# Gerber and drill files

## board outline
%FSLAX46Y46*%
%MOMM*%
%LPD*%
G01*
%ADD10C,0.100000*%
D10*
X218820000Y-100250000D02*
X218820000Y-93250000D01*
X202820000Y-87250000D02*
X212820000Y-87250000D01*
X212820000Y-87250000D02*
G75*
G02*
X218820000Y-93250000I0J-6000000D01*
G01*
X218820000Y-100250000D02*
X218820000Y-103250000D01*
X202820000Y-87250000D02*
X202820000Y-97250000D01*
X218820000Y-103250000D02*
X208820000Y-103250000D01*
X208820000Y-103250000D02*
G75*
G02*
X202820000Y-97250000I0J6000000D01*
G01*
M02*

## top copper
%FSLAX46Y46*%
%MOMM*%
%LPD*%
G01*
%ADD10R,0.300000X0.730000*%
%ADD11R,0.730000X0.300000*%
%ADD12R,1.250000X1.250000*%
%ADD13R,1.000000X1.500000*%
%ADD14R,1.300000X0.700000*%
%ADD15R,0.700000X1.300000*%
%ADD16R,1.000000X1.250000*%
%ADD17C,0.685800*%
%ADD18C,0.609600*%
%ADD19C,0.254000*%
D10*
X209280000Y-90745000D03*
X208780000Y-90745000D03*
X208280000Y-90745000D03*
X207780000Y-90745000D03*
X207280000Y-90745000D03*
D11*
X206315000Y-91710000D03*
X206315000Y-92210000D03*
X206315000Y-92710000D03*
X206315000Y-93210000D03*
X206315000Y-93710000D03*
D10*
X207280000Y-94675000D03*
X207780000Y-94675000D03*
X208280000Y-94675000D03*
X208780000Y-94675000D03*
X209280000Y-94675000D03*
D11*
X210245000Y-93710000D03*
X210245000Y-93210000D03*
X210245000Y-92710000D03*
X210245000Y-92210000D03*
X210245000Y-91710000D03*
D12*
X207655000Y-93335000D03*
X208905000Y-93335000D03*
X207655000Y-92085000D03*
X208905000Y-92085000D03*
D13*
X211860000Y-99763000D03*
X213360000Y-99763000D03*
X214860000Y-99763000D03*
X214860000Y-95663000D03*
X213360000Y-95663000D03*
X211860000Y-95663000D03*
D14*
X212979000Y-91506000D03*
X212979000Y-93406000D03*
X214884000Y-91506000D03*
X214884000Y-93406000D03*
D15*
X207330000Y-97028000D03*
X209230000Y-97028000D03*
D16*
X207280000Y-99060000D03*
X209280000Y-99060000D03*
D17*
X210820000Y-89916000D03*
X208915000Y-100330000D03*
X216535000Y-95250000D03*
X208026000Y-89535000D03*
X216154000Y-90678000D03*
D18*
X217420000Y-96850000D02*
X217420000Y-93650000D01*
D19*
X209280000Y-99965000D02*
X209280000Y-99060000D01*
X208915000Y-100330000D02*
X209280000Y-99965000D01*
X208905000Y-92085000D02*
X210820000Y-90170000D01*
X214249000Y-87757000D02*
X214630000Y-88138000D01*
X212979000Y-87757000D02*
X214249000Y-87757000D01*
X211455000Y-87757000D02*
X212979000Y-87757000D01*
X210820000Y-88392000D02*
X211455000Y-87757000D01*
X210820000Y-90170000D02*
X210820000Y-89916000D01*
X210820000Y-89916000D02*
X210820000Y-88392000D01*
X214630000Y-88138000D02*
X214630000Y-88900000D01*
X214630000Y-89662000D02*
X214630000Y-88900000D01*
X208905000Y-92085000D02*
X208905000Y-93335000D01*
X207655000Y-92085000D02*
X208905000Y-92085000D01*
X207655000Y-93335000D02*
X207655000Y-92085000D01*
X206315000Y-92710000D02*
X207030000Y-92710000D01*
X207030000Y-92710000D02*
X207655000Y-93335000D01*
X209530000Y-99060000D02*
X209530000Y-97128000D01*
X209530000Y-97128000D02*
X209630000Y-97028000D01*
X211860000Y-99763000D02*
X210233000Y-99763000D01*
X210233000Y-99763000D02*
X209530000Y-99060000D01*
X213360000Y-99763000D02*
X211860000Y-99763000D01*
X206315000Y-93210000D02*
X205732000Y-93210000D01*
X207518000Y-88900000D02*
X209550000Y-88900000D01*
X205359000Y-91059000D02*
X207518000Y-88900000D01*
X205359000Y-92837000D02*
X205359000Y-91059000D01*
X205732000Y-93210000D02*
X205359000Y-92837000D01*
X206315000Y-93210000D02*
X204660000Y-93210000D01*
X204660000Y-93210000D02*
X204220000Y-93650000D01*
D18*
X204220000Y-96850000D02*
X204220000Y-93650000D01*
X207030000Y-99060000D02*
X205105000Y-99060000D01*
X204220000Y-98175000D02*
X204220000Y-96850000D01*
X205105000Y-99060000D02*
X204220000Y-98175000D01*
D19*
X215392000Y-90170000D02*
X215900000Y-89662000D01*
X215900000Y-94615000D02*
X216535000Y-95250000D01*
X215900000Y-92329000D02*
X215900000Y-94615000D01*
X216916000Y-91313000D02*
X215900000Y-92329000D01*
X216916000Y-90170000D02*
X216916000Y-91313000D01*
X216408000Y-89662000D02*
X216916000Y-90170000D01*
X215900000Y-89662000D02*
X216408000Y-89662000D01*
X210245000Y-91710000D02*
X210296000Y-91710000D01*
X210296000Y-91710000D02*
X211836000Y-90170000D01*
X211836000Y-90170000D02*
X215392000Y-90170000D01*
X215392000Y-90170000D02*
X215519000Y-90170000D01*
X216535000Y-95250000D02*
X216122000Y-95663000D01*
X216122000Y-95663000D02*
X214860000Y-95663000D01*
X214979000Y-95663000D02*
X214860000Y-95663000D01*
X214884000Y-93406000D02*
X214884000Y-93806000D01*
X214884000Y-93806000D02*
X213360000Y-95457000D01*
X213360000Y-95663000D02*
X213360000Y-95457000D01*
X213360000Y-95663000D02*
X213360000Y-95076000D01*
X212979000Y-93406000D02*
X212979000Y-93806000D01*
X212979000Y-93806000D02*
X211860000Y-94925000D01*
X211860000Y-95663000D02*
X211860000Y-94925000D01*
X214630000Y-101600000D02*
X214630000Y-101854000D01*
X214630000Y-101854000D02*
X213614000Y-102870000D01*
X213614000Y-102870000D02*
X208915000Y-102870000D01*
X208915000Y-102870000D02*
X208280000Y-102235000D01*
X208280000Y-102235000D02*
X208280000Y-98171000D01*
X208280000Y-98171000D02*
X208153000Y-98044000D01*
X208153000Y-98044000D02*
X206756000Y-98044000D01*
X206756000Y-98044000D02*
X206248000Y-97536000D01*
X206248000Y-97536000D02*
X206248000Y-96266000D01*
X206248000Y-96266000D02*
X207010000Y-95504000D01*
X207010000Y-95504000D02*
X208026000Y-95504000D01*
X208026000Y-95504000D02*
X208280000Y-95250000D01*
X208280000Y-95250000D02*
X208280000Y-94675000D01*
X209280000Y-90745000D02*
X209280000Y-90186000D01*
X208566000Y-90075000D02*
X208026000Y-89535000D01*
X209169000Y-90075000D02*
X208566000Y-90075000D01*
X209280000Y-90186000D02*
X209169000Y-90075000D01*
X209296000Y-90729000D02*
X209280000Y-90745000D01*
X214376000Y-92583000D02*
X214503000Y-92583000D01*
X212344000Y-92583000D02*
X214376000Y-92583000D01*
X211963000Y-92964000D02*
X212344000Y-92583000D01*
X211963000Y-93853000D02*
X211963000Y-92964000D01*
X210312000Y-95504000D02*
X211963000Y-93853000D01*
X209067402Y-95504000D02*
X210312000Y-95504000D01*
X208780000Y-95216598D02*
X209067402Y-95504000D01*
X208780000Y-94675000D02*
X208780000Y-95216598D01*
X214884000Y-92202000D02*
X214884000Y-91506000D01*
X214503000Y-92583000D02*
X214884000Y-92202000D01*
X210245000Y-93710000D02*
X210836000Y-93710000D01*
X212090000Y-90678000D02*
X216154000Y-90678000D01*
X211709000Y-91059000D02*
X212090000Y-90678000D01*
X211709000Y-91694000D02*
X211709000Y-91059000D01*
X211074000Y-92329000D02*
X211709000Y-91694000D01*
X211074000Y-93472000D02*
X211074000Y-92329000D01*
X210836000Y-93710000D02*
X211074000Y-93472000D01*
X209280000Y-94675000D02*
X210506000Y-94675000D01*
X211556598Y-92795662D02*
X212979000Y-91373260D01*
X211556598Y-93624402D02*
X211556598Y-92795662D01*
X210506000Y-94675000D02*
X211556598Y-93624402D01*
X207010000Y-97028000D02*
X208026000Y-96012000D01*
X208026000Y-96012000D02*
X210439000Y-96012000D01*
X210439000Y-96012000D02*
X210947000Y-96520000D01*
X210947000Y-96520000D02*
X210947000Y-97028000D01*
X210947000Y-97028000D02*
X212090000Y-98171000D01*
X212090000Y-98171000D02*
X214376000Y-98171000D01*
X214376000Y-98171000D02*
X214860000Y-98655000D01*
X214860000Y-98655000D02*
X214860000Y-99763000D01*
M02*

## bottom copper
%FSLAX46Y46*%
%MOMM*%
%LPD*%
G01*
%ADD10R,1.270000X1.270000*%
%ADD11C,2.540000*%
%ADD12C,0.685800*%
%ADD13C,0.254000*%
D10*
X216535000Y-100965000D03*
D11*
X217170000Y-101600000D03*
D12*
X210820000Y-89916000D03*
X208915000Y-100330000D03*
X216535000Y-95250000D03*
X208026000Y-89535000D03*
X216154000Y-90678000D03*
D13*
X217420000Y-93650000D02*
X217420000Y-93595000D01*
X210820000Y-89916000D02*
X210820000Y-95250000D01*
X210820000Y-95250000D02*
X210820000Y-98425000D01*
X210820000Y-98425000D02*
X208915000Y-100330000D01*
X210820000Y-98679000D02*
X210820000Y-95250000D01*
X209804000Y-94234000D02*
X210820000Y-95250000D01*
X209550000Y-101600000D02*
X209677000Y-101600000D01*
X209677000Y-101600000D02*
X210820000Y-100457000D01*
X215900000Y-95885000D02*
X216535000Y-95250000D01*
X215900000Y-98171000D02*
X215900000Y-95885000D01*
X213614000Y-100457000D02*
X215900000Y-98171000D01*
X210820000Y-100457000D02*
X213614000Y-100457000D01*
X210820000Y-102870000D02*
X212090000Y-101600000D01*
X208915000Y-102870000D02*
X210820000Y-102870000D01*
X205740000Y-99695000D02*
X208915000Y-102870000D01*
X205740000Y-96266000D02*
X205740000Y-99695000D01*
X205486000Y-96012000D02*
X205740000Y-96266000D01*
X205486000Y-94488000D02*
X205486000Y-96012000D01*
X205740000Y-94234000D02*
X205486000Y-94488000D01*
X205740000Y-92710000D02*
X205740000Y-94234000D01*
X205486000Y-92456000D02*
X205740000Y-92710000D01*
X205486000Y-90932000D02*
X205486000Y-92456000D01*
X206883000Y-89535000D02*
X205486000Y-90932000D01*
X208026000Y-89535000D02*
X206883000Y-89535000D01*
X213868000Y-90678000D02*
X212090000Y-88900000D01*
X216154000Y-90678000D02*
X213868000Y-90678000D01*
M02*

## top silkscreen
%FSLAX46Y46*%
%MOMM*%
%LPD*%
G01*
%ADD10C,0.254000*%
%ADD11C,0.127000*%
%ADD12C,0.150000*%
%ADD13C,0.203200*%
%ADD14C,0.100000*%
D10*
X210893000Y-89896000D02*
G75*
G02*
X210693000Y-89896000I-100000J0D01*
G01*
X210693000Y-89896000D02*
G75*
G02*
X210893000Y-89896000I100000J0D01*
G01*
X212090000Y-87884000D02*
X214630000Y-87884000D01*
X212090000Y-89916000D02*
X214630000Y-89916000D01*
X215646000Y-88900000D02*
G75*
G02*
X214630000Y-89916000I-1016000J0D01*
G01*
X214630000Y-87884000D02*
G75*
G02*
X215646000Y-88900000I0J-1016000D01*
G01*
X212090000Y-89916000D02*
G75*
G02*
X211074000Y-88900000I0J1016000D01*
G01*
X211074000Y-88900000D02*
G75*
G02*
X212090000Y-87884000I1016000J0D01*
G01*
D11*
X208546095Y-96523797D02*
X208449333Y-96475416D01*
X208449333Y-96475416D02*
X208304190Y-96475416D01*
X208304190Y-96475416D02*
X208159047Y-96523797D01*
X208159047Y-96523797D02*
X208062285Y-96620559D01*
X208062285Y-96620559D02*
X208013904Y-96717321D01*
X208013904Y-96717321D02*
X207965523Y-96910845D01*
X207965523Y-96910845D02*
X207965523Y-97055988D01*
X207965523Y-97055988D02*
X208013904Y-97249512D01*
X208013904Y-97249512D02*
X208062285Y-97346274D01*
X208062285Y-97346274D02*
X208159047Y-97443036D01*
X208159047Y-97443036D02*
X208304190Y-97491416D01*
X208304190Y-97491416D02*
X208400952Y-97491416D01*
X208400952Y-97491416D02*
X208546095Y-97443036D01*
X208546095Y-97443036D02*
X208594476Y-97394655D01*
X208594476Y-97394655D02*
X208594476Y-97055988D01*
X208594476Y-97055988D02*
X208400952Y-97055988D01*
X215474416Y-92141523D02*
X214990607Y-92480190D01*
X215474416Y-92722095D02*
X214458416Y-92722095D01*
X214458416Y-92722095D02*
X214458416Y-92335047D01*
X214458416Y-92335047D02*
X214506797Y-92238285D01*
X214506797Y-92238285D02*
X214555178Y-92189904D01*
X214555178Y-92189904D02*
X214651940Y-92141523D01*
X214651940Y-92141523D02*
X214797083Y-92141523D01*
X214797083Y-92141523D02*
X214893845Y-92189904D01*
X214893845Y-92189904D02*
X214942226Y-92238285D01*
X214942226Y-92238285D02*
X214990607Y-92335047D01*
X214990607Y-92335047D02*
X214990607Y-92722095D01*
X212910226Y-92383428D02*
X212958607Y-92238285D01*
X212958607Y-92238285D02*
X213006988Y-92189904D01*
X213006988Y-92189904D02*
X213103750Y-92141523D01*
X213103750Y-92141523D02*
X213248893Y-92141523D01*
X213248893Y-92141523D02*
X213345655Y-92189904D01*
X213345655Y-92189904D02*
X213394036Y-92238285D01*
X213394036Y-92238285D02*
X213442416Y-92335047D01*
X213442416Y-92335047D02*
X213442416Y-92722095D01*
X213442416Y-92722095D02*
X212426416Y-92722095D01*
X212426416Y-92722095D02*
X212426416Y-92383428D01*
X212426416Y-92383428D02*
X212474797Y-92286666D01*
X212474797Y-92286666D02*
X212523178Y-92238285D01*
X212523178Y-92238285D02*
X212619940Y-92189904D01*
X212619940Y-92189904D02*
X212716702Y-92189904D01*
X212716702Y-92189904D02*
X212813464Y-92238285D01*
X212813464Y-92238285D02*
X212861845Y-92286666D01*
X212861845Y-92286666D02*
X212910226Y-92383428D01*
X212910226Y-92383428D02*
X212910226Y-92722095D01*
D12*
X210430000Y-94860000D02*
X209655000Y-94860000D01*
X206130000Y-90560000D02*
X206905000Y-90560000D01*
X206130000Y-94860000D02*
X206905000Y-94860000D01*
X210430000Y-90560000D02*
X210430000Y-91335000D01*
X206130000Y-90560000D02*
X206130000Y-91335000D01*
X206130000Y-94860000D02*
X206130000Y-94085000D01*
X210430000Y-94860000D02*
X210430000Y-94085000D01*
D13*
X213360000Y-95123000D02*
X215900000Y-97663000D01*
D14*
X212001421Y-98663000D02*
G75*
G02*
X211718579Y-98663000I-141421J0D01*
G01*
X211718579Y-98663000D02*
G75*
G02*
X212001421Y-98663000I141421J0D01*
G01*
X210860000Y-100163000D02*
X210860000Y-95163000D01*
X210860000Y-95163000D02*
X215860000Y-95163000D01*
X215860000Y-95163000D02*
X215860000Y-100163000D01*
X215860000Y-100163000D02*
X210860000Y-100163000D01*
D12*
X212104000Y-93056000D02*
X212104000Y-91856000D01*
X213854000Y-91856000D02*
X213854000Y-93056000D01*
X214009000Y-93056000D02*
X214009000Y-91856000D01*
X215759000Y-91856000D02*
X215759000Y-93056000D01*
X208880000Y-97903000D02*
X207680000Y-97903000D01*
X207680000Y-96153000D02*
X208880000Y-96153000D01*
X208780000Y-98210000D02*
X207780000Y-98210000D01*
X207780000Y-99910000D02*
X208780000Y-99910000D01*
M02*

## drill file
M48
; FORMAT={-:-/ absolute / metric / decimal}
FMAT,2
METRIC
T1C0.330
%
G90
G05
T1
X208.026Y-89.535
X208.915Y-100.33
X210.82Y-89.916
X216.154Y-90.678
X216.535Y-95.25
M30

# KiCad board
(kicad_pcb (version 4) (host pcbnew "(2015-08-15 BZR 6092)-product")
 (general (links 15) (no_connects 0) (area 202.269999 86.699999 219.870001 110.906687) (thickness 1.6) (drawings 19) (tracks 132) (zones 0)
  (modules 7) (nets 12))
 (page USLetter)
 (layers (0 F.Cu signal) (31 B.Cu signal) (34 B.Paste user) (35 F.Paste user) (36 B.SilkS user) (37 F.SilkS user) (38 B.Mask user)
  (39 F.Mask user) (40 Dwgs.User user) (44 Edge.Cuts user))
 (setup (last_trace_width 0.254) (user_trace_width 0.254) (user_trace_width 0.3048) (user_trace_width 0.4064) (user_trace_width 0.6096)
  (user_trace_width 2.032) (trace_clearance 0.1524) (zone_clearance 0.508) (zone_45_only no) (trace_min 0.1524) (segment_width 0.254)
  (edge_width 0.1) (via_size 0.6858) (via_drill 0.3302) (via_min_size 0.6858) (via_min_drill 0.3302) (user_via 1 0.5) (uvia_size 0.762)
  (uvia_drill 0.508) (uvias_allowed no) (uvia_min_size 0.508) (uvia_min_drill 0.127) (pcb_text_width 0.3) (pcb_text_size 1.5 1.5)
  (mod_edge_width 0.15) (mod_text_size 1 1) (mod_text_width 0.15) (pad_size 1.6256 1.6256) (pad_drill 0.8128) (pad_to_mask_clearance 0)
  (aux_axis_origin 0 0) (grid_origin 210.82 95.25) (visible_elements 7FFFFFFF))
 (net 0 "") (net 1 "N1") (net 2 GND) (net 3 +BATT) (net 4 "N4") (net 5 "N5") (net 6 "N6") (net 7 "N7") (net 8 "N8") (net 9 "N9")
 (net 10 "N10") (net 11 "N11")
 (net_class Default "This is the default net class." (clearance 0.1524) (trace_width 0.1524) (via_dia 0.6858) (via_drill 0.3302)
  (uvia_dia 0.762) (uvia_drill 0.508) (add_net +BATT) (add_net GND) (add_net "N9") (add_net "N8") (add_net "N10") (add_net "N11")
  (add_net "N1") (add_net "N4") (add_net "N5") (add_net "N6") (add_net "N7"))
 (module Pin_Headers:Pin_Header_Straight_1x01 (layer B.Cu) (at 216.535 100.965 270)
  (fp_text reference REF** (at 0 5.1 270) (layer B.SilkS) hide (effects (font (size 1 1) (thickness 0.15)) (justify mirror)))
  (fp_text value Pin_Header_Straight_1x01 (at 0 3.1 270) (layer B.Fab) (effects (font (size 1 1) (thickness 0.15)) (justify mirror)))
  (pad 1 smd rect (at 0 0 270) (size 1.27 1.27) (layers B.Cu B.Paste B.Mask))
  (pad 1 smd circle (at 0.635 -0.635 270) (size 2.54 2.54) (layers B.Cu B.Paste B.Mask)))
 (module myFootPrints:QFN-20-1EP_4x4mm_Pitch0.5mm (layer F.Cu) (at 208.28 92.71 270)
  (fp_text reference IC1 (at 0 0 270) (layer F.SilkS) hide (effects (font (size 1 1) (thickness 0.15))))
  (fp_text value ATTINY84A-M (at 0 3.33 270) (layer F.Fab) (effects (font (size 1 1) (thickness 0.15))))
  (fp_line (start 2.15 -2.15) (end 2.15 -1.375) (layer F.SilkS) (width 0.15))
  (fp_line (start -2.15 2.15) (end -2.15 1.375) (layer F.SilkS) (width 0.15))
  (fp_line (start 2.15 2.15) (end 2.15 1.375) (layer F.SilkS) (width 0.15))
  (fp_line (start -2.15 -2.15) (end -1.375 -2.15) (layer F.SilkS) (width 0.15))
  (fp_line (start -2.15 2.15) (end -1.375 2.15) (layer F.SilkS) (width 0.15))
  (fp_line (start 2.15 2.15) (end 1.375 2.15) (layer F.SilkS) (width 0.15))
  (fp_line (start 2.15 -2.15) (end 1.375 -2.15) (layer F.SilkS) (width 0.15))
  (pad 1 smd rect (at -1.965 -1 270) (size 0.73 0.3) (layers F.Cu F.Paste F.Mask) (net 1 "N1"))
  (pad 2 smd rect (at -1.965 -0.5 270) (size 0.73 0.3) (layers F.Cu F.Paste F.Mask))
  (pad 3 smd rect (at -1.965 0 270) (size 0.73 0.3) (layers F.Cu F.Paste F.Mask))
  (pad 4 smd rect (at -1.965 0.5 270) (size 0.73 0.3) (layers F.Cu F.Paste F.Mask))
  (pad 5 smd rect (at -1.965 1 270) (size 0.73 0.3) (layers F.Cu F.Paste F.Mask))
  (pad 6 smd rect (at -1 1.965) (size 0.73 0.3) (layers F.Cu F.Paste F.Mask))
  (pad 7 smd rect (at -0.5 1.965) (size 0.73 0.3) (layers F.Cu F.Paste F.Mask))
  (pad 8 smd rect (at 0 1.965) (size 0.73 0.3) (layers F.Cu F.Paste F.Mask) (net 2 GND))
  (pad 9 smd rect (at 0.5 1.965) (size 0.73 0.3) (layers F.Cu F.Paste F.Mask) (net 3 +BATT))
  (pad 10 smd rect (at 1 1.965) (size 0.73 0.3) (layers F.Cu F.Paste F.Mask))
  (pad 11 smd rect (at 1.965 1 270) (size 0.73 0.3) (layers F.Cu F.Paste F.Mask))
  (pad 12 smd rect (at 1.965 0.5 270) (size 0.73 0.3) (layers F.Cu F.Paste F.Mask))
  (pad 13 smd rect (at 1.965 0 270) (size 0.73 0.3) (layers F.Cu F.Paste F.Mask) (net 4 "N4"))
  (pad 14 smd rect (at 1.965 -0.5 270) (size 0.73 0.3) (layers F.Cu F.Paste F.Mask) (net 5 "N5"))
  (pad 15 smd rect (at 1.965 -1 270) (size 0.73 0.3) (layers F.Cu F.Paste F.Mask) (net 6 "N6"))
  (pad 16 smd rect (at 1 -1.965) (size 0.73 0.3) (layers F.Cu F.Paste F.Mask) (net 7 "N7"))
  (pad 17 smd rect (at 0.5 -1.965) (size 0.73 0.3) (layers F.Cu F.Paste F.Mask))
  (pad 18 smd rect (at 0 -1.965) (size 0.73 0.3) (layers F.Cu F.Paste F.Mask))
  (pad 19 smd rect (at -0.5 -1.965) (size 0.73 0.3) (layers F.Cu F.Paste F.Mask))
  (pad 20 smd rect (at -1 -1.965) (size 0.73 0.3) (layers F.Cu F.Paste F.Mask) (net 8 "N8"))
  (pad 8 smd rect (at 0.625 0.625 270) (size 1.25 1.25) (layers F.Cu F.Paste F.Mask) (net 2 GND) (solder_paste_margin_ratio -0.2))
  (pad 8 smd rect (at 0.625 -0.625 270) (size 1.25 1.25) (layers F.Cu F.Paste F.Mask) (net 2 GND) (solder_paste_margin_ratio -0.2))
  (pad 8 smd rect (at -0.625 0.625 270) (size 1.25 1.25) (layers F.Cu F.Paste F.Mask) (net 2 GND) (solder_paste_margin_ratio -0.2))
  (pad 8 smd rect (at -0.625 -0.625 270) (size 1.25 1.25) (layers F.Cu F.Paste F.Mask) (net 2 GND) (solder_paste_margin_ratio -0.2)))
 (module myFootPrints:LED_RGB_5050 (layer F.Cu) (at 213.36 97.663 90)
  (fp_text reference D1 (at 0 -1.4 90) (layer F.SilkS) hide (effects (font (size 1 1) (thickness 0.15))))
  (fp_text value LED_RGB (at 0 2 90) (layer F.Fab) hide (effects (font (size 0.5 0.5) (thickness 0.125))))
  (fp_line (start 2.54 0) (end 0 2.54) (layer F.SilkS) (width 0.2032))
  (fp_circle (center -1 -1.5) (end -1.1 -1.6) (layer F.SilkS) (width 0.1))
  (fp_line (start -2.5 -2.5) (end 2.5 -2.5) (layer F.SilkS) (width 0.1))
  (fp_line (start 2.5 -2.5) (end 2.5 2.5) (layer F.SilkS) (width 0.1))
  (fp_line (start 2.5 2.5) (end -2.5 2.5) (layer F.SilkS) (width 0.1))
  (fp_line (start -2.5 2.5) (end -2.5 -2.5) (layer F.SilkS) (width 0.1))
  (pad 1 smd rect (at -2.1 -1.5 180) (size 1 1.5) (layers F.Cu F.Paste F.Mask) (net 2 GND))
  (pad 2 smd rect (at -2.1 0 180) (size 1 1.5) (layers F.Cu F.Paste F.Mask) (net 2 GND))
  (pad 3 smd rect (at -2.1 1.5 180) (size 1 1.5) (layers F.Cu F.Paste F.Mask) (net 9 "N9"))
  (pad 4 smd rect (at 2 1.5 180) (size 1 1.5) (layers F.Cu F.Paste F.Mask) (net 8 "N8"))
  (pad 5 smd rect (at 2 0 180) (size 1 1.5) (layers F.Cu F.Paste F.Mask) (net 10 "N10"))
  (pad 6 smd rect (at 2 -1.5 180) (size 1 1.5) (layers F.Cu F.Paste F.Mask) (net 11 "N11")))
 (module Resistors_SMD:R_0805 (layer F.Cu) (at 212.979 92.456 270)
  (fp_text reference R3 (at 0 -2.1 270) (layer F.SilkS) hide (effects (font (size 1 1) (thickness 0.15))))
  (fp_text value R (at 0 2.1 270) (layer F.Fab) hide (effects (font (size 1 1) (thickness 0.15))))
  (fp_line (start 0.6 0.875) (end -0.6 0.875) (layer F.SilkS) (width 0.15))
  (fp_line (start -0.6 -0.875) (end 0.6 -0.875) (layer F.SilkS) (width 0.15))
  (pad 1 smd rect (at -0.95 0 270) (size 0.7 1.3) (layers F.Cu F.Paste F.Mask) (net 6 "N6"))
  (pad 2 smd rect (at 0.95 0 270) (size 0.7 1.3) (layers F.Cu F.Paste F.Mask) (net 11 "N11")))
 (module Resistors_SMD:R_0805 (layer F.Cu) (at 214.884 92.456 270)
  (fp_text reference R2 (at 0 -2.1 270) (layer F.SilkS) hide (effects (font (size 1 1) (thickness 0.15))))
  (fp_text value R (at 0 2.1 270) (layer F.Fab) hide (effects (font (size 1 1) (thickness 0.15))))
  (fp_line (start 0.6 0.875) (end -0.6 0.875) (layer F.SilkS) (width 0.15))
  (fp_line (start -0.6 -0.875) (end 0.6 -0.875) (layer F.SilkS) (width 0.15))
  (pad 1 smd rect (at -0.95 0 270) (size 0.7 1.3) (layers F.Cu F.Paste F.Mask) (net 5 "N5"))
  (pad 2 smd rect (at 0.95 0 270) (size 0.7 1.3) (layers F.Cu F.Paste F.Mask) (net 10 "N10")))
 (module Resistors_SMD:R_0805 (layer F.Cu) (at 208.28 97.028)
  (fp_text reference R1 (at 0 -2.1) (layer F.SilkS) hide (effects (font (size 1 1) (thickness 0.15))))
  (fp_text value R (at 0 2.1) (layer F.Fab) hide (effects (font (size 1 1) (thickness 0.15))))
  (fp_line (start 0.6 0.875) (end -0.6 0.875) (layer F.SilkS) (width 0.15))
  (fp_line (start -0.6 -0.875) (end 0.6 -0.875) (layer F.SilkS) (width 0.15))
  (pad 1 smd rect (at -0.95 0) (size 0.7 1.3) (layers F.Cu F.Paste F.Mask) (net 9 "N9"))
  (pad 2 smd rect (at 0.95 0) (size 0.7 1.3) (layers F.Cu F.Paste F.Mask) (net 2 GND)))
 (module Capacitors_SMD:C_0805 (layer F.Cu) (at 208.28 99.06)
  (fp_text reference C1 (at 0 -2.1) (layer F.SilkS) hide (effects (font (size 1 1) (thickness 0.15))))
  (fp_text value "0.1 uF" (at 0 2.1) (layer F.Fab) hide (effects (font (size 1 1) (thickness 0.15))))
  (fp_line (start 0.5 -0.85) (end -0.5 -0.85) (layer F.SilkS) (width 0.15))
  (fp_line (start -0.5 0.85) (end 0.5 0.85) (layer F.SilkS) (width 0.15))
  (pad 1 smd rect (at -1 0) (size 1 1.25) (layers F.Cu F.Paste F.Mask) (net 3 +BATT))
  (pad 2 smd rect (at 1 0) (size 1 1.25) (layers F.Cu F.Paste F.Mask) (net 2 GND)))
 (gr_line (start 218.82 100.25) (end 218.82 93.25) (angle 90) (layer Edge.Cuts) (width 0.1))
 (gr_line (start 202.82 87.25) (end 212.82 87.25) (angle 90) (layer Edge.Cuts) (width 0.1))
 (gr_arc (start 212.82 93.25) (end 212.82 87.25) (angle 90) (layer Edge.Cuts) (width 0.1))
 (gr_line (start 218.82 100.25) (end 218.82 103.25) (angle 90) (layer Edge.Cuts) (width 0.1))
 (gr_line (start 202.82 87.25) (end 202.82 97.25) (angle 90) (layer Edge.Cuts) (width 0.1))
 (gr_line (start 218.82 103.25) (end 208.82 103.25) (angle 90) (layer Edge.Cuts) (width 0.1))
 (gr_arc (start 208.82 97.25) (end 208.82 103.25) (angle 90) (layer Edge.Cuts) (width 0.1))
 (gr_circle (center 210.793 89.896) (end 210.893 89.896) (layer F.SilkS) (width 0.254))
 (gr_line (start 212.09 87.884) (end 214.63 87.884) (angle 90) (layer F.SilkS) (width 0.254))
 (gr_line (start 212.09 89.916) (end 214.63 89.916) (angle 90) (layer F.SilkS) (width 0.254))
 (gr_arc (start 214.63 88.9) (end 215.646 88.9) (angle 90) (layer F.SilkS) (width 0.254))
 (gr_arc (start 214.63 88.9) (end 214.63 87.884) (angle 90) (layer F.SilkS) (width 0.254))
 (gr_arc (start 212.09 88.9) (end 212.09 89.916) (angle 90) (layer F.SilkS) (width 0.254))
 (gr_arc (start 212.09 88.9) (end 211.074 88.9) (angle 90) (layer F.SilkS) (width 0.254))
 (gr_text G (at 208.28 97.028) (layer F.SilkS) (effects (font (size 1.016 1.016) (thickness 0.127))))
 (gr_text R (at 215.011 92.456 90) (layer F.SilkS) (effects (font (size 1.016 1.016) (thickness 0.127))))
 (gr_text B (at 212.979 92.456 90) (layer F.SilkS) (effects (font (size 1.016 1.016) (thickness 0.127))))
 (segment (start 217.42 93.65) (end 217.42 93.595) (width 0.254) (layer B.Cu) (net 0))
 (segment (start 217.42 96.85) (end 217.42 93.65) (width 0.6096) (layer F.Cu) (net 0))
 (via (at 210.82 89.916) (size 0.6858) (drill 0.3302) (layers F.Cu B.Cu) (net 2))
 (segment (start 210.82 89.916) (end 210.82 95.25) (width 0.254) (layer B.Cu) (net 2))
 (segment (start 210.82 95.25) (end 210.82 98.425) (width 0.254) (layer B.Cu) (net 2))
 (segment (start 210.82 98.425) (end 208.915 100.33) (width 0.254) (layer B.Cu) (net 2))
 (segment (start 209.28 99.965) (end 209.28 99.06) (width 0.254) (layer F.Cu) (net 2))
 (segment (start 208.915 100.33) (end 209.28 99.965) (width 0.254) (layer F.Cu) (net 2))
 (via (at 208.915 100.33) (size 0.6858) (drill 0.3302) (layers F.Cu B.Cu) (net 2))
 (segment (start 208.905 92.085) (end 210.82 90.17) (width 0.254) (layer F.Cu) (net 2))
 (segment (start 214.249 87.757) (end 214.63 88.138) (width 0.254) (layer F.Cu) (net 2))
 (segment (start 212.979 87.757) (end 214.249 87.757) (width 0.254) (layer F.Cu) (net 2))
 (segment (start 211.455 87.757) (end 212.979 87.757) (width 0.254) (layer F.Cu) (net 2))
 (segment (start 210.82 88.392) (end 211.455 87.757) (width 0.254) (layer F.Cu) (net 2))
 (segment (start 210.82 90.17) (end 210.82 89.916) (width 0.254) (layer F.Cu) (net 2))
 (segment (start 210.82 89.916) (end 210.82 88.392) (width 0.254) (layer F.Cu) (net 2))
 (segment (start 214.63 88.138) (end 214.63 88.9) (width 0.254) (layer F.Cu) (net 2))
 (segment (start 214.63 89.662) (end 214.63 88.9) (width 0.254) (layer F.Cu) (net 2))
 (segment (start 208.905 92.085) (end 208.905 93.335) (width 0.254) (layer F.Cu) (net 2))
 (segment (start 207.655 92.085) (end 208.905 92.085) (width 0.254) (layer F.Cu) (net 2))
 (segment (start 207.655 93.335) (end 207.655 92.085) (width 0.254) (layer F.Cu) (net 2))
 (segment (start 206.315 92.71) (end 207.03 92.71) (width 0.254) (layer F.Cu) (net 2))
 (segment (start 207.03 92.71) (end 207.655 93.335) (width 0.254) (layer F.Cu) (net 2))
 (segment (start 210.82 98.679) (end 210.82 95.25) (width 0.254) (layer B.Cu) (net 2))
 (segment (start 209.804 94.234) (end 210.82 95.25) (width 0.254) (layer B.Cu) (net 2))
 (segment (start 209.53 99.06) (end 209.53 97.128) (width 0.254) (layer F.Cu) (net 2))
 (segment (start 209.53 97.128) (end 209.63 97.028) (width 0.254) (layer F.Cu) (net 2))
 (segment (start 211.86 99.763) (end 210.233 99.763) (width 0.254) (layer F.Cu) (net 2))
 (segment (start 210.233 99.763) (end 209.53 99.06) (width 0.254) (layer F.Cu) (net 2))
 (segment (start 213.36 99.763) (end 211.86 99.763) (width 0.254) (layer F.Cu) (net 2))
 (segment (start 206.315 93.21) (end 205.732 93.21) (width 0.254) (layer F.Cu) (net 3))
 (segment (start 207.518 88.9) (end 209.55 88.9) (width 0.254) (layer F.Cu) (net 3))
 (segment (start 205.359 91.059) (end 207.518 88.9) (width 0.254) (layer F.Cu) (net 3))
 (segment (start 205.359 92.837) (end 205.359 91.059) (width 0.254) (layer F.Cu) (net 3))
 (segment (start 205.732 93.21) (end 205.359 92.837) (width 0.254) (layer F.Cu) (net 3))
 (segment (start 206.315 93.21) (end 204.66 93.21) (width 0.254) (layer F.Cu) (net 3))
 (segment (start 204.66 93.21) (end 204.22 93.65) (width 0.254) (layer F.Cu) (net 3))
 (segment (start 204.22 96.85) (end 204.22 93.65) (width 0.6096) (layer F.Cu) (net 3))
 (segment (start 207.03 99.06) (end 205.105 99.06) (width 0.6096) (layer F.Cu) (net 3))
 (segment (start 204.22 98.175) (end 204.22 96.85) (width 0.6096) (layer F.Cu) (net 3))
 (segment (start 205.105 99.06) (end 204.22 98.175) (width 0.6096) (layer F.Cu) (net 3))
 (segment (start 215.392 90.17) (end 215.9 89.662) (width 0.254) (layer F.Cu) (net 8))
 (segment (start 215.9 94.615) (end 216.535 95.25) (width 0.254) (layer F.Cu) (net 8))
 (segment (start 215.9 92.329) (end 215.9 94.615) (width 0.254) (layer F.Cu) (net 8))
 (segment (start 216.916 91.313) (end 215.9 92.329) (width 0.254) (layer F.Cu) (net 8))
 (segment (start 216.916 90.17) (end 216.916 91.313) (width 0.254) (layer F.Cu) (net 8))
 (segment (start 216.408 89.662) (end 216.916 90.17) (width 0.254) (layer F.Cu) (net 8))
 (segment (start 215.9 89.662) (end 216.408 89.662) (width 0.254) (layer F.Cu) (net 8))
 (segment (start 210.245 91.71) (end 210.296 91.71) (width 0.254) (layer F.Cu) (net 8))
 (segment (start 210.296 91.71) (end 211.836 90.17) (width 0.254) (layer F.Cu) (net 8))
 (segment (start 211.836 90.17) (end 215.392 90.17) (width 0.254) (layer F.Cu) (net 8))
 (segment (start 215.392 90.17) (end 215.519 90.17) (width 0.254) (layer F.Cu) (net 8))
 (segment (start 209.55 101.6) (end 209.677 101.6) (width 0.254) (layer B.Cu) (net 8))
 (segment (start 209.677 101.6) (end 210.82 100.457) (width 0.254) (layer B.Cu) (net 8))
 (via (at 216.535 95.25) (size 0.6858) (drill 0.3302) (layers F.Cu B.Cu) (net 8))
 (segment (start 215.9 95.885) (end 216.535 95.25) (width 0.254) (layer B.Cu) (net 8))
 (segment (start 215.9 98.171) (end 215.9 95.885) (width 0.254) (layer B.Cu) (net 8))
 (segment (start 213.614 100.457) (end 215.9 98.171) (width 0.254) (layer B.Cu) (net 8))
 (segment (start 210.82 100.457) (end 213.614 100.457) (width 0.254) (layer B.Cu) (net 8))
 (segment (start 216.535 95.25) (end 216.122 95.663) (width 0.254) (layer F.Cu) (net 8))
 (segment (start 216.122 95.663) (end 214.86 95.663) (width 0.254) (layer F.Cu) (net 8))
 (segment (start 214.979 95.663) (end 214.86 95.663) (width 0.254) (layer F.Cu) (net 8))
 (segment (start 214.884 93.406) (end 214.884 93.806) (width 0.254) (layer F.Cu) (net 10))
 (segment (start 214.884 93.806) (end 213.36 95.457) (width 0.254) (layer F.Cu) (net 10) (status 20))
 (segment (start 213.36 95.663) (end 213.36 95.457) (width 0.254) (layer F.Cu) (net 10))
 (segment (start 213.36 95.663) (end 213.36 95.076) (width 0.254) (layer F.Cu) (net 10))
 (segment (start 212.979 93.406) (end 212.979 93.806) (width 0.254) (layer F.Cu) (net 11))
 (segment (start 212.979 93.806) (end 211.86 94.925) (width 0.254) (layer F.Cu) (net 11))
 (segment (start 211.86 95.663) (end 211.86 94.925) (width 0.254) (layer F.Cu) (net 11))
 (segment (start 214.63 101.6) (end 214.63 101.854) (width 0.254) (layer F.Cu) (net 4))
 (segment (start 214.63 101.854) (end 213.614 102.87) (width 0.254) (layer F.Cu) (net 4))
 (segment (start 213.614 102.87) (end 208.915 102.87) (width 0.254) (layer F.Cu) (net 4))
 (segment (start 208.915 102.87) (end 208.28 102.235) (width 0.254) (layer F.Cu) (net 4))
 (segment (start 208.28 102.235) (end 208.28 98.171) (width 0.254) (layer F.Cu) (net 4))
 (segment (start 208.28 98.171) (end 208.153 98.044) (width 0.254) (layer F.Cu) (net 4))
 (segment (start 208.153 98.044) (end 206.756 98.044) (width 0.254) (layer F.Cu) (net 4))
 (segment (start 206.756 98.044) (end 206.248 97.536) (width 0.254) (layer F.Cu) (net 4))
 (segment (start 206.248 97.536) (end 206.248 96.266) (width 0.254) (layer F.Cu) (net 4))
 (segment (start 206.248 96.266) (end 207.01 95.504) (width 0.254) (layer F.Cu) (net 4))
 (segment (start 207.01 95.504) (end 208.026 95.504) (width 0.254) (layer F.Cu) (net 4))
 (segment (start 208.026 95.504) (end 208.28 95.25) (width 0.254) (layer F.Cu) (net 4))
 (segment (start 208.28 95.25) (end 208.28 94.675) (width 0.254) (layer F.Cu) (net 4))
 (segment (start 209.28 90.745) (end 209.28 90.186) (width 0.254) (layer F.Cu) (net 1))
 (segment (start 210.82 102.87) (end 212.09 101.6) (width 0.254) (layer B.Cu) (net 1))
 (segment (start 208.915 102.87) (end 210.82 102.87) (width 0.254) (layer B.Cu) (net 1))
 (segment (start 205.74 99.695) (end 208.915 102.87) (width 0.254) (layer B.Cu) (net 1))
 (segment (start 205.74 96.266) (end 205.74 99.695) (width 0.254) (layer B.Cu) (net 1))
 (segment (start 205.486 96.012) (end 205.74 96.266) (width 0.254) (layer B.Cu) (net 1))
 (segment (start 205.486 94.488) (end 205.486 96.012) (width 0.254) (layer B.Cu) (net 1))
 (segment (start 205.74 94.234) (end 205.486 94.488) (width 0.254) (layer B.Cu) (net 1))
 (segment (start 205.74 92.71) (end 205.74 94.234) (width 0.254) (layer B.Cu) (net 1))
 (segment (start 205.486 92.456) (end 205.74 92.71) (width 0.254) (layer B.Cu) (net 1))
 (segment (start 205.486 90.932) (end 205.486 92.456) (width 0.254) (layer B.Cu) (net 1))
 (segment (start 206.883 89.535) (end 205.486 90.932) (width 0.254) (layer B.Cu) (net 1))
 (segment (start 208.026 89.535) (end 206.883 89.535) (width 0.254) (layer B.Cu) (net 1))
 (via (at 208.026 89.535) (size 0.6858) (drill 0.3302) (layers F.Cu B.Cu) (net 1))
 (segment (start 208.566 90.075) (end 208.026 89.535) (width 0.254) (layer F.Cu) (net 1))
 (segment (start 209.169 90.075) (end 208.566 90.075) (width 0.254) (layer F.Cu) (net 1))
 (segment (start 209.28 90.186) (end 209.169 90.075) (width 0.254) (layer F.Cu) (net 1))
 (segment (start 209.296 90.729) (end 209.28 90.745) (width 0.254) (layer F.Cu) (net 1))
 (segment (start 214.376 92.583) (end 214.503 92.583) (width 0.254) (layer F.Cu) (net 5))
 (segment (start 212.344 92.583) (end 214.376 92.583) (width 0.254) (layer F.Cu) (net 5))
 (segment (start 211.963 92.964) (end 212.344 92.583) (width 0.254) (layer F.Cu) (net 5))
 (segment (start 211.963 93.853) (end 211.963 92.964) (width 0.254) (layer F.Cu) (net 5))
 (segment (start 210.312 95.504) (end 211.963 93.853) (width 0.254) (layer F.Cu) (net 5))
 (segment (start 209.067402 95.504) (end 210.312 95.504) (width 0.254) (layer F.Cu) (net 5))
 (segment (start 208.78 95.216598) (end 209.067402 95.504) (width 0.254) (layer F.Cu) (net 5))
 (segment (start 208.78 94.675) (end 208.78 95.216598) (width 0.254) (layer F.Cu) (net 5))
 (segment (start 214.884 92.202) (end 214.884 91.506) (width 0.254) (layer F.Cu) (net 5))
 (segment (start 214.503 92.583) (end 214.884 92.202) (width 0.254) (layer F.Cu) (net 5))
 (segment (start 210.245 93.71) (end 210.836 93.71) (width 0.254) (layer F.Cu) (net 7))
 (segment (start 213.868 90.678) (end 212.09 88.9) (width 0.254) (layer B.Cu) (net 7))
 (segment (start 216.154 90.678) (end 213.868 90.678) (width 0.254) (layer B.Cu) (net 7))
 (via (at 216.154 90.678) (size 0.6858) (drill 0.3302) (layers F.Cu B.Cu) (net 7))
 (segment (start 212.09 90.678) (end 216.154 90.678) (width 0.254) (layer F.Cu) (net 7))
 (segment (start 211.709 91.059) (end 212.09 90.678) (width 0.254) (layer F.Cu) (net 7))
 (segment (start 211.709 91.694) (end 211.709 91.059) (width 0.254) (layer F.Cu) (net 7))
 (segment (start 211.074 92.329) (end 211.709 91.694) (width 0.254) (layer F.Cu) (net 7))
 (segment (start 211.074 93.472) (end 211.074 92.329) (width 0.254) (layer F.Cu) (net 7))
 (segment (start 210.836 93.71) (end 211.074 93.472) (width 0.254) (layer F.Cu) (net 7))
 (segment (start 209.28 94.675) (end 210.506 94.675) (width 0.254) (layer F.Cu) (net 6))
 (segment (start 211.556598 92.795662) (end 212.979 91.37326) (width 0.254) (layer F.Cu) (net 6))
 (segment (start 211.556598 93.624402) (end 211.556598 92.795662) (width 0.254) (layer F.Cu) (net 6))
 (segment (start 210.506 94.675) (end 211.556598 93.624402) (width 0.254) (layer F.Cu) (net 6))
 (segment (start 207.01 97.028) (end 208.026 96.012) (width 0.254) (layer F.Cu) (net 9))
 (segment (start 208.026 96.012) (end 210.439 96.012) (width 0.254) (layer F.Cu) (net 9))
 (segment (start 210.439 96.012) (end 210.947 96.52) (width 0.254) (layer F.Cu) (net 9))
 (segment (start 210.947 96.52) (end 210.947 97.028) (width 0.254) (layer F.Cu) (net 9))
 (segment (start 210.947 97.028) (end 212.09 98.171) (width 0.254) (layer F.Cu) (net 9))
 (segment (start 212.09 98.171) (end 214.376 98.171) (width 0.254) (layer F.Cu) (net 9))
 (segment (start 214.376 98.171) (end 214.86 98.655) (width 0.254) (layer F.Cu) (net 9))
 (segment (start 214.86 98.655) (end 214.86 99.763) (width 0.254) (layer F.Cu) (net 9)))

